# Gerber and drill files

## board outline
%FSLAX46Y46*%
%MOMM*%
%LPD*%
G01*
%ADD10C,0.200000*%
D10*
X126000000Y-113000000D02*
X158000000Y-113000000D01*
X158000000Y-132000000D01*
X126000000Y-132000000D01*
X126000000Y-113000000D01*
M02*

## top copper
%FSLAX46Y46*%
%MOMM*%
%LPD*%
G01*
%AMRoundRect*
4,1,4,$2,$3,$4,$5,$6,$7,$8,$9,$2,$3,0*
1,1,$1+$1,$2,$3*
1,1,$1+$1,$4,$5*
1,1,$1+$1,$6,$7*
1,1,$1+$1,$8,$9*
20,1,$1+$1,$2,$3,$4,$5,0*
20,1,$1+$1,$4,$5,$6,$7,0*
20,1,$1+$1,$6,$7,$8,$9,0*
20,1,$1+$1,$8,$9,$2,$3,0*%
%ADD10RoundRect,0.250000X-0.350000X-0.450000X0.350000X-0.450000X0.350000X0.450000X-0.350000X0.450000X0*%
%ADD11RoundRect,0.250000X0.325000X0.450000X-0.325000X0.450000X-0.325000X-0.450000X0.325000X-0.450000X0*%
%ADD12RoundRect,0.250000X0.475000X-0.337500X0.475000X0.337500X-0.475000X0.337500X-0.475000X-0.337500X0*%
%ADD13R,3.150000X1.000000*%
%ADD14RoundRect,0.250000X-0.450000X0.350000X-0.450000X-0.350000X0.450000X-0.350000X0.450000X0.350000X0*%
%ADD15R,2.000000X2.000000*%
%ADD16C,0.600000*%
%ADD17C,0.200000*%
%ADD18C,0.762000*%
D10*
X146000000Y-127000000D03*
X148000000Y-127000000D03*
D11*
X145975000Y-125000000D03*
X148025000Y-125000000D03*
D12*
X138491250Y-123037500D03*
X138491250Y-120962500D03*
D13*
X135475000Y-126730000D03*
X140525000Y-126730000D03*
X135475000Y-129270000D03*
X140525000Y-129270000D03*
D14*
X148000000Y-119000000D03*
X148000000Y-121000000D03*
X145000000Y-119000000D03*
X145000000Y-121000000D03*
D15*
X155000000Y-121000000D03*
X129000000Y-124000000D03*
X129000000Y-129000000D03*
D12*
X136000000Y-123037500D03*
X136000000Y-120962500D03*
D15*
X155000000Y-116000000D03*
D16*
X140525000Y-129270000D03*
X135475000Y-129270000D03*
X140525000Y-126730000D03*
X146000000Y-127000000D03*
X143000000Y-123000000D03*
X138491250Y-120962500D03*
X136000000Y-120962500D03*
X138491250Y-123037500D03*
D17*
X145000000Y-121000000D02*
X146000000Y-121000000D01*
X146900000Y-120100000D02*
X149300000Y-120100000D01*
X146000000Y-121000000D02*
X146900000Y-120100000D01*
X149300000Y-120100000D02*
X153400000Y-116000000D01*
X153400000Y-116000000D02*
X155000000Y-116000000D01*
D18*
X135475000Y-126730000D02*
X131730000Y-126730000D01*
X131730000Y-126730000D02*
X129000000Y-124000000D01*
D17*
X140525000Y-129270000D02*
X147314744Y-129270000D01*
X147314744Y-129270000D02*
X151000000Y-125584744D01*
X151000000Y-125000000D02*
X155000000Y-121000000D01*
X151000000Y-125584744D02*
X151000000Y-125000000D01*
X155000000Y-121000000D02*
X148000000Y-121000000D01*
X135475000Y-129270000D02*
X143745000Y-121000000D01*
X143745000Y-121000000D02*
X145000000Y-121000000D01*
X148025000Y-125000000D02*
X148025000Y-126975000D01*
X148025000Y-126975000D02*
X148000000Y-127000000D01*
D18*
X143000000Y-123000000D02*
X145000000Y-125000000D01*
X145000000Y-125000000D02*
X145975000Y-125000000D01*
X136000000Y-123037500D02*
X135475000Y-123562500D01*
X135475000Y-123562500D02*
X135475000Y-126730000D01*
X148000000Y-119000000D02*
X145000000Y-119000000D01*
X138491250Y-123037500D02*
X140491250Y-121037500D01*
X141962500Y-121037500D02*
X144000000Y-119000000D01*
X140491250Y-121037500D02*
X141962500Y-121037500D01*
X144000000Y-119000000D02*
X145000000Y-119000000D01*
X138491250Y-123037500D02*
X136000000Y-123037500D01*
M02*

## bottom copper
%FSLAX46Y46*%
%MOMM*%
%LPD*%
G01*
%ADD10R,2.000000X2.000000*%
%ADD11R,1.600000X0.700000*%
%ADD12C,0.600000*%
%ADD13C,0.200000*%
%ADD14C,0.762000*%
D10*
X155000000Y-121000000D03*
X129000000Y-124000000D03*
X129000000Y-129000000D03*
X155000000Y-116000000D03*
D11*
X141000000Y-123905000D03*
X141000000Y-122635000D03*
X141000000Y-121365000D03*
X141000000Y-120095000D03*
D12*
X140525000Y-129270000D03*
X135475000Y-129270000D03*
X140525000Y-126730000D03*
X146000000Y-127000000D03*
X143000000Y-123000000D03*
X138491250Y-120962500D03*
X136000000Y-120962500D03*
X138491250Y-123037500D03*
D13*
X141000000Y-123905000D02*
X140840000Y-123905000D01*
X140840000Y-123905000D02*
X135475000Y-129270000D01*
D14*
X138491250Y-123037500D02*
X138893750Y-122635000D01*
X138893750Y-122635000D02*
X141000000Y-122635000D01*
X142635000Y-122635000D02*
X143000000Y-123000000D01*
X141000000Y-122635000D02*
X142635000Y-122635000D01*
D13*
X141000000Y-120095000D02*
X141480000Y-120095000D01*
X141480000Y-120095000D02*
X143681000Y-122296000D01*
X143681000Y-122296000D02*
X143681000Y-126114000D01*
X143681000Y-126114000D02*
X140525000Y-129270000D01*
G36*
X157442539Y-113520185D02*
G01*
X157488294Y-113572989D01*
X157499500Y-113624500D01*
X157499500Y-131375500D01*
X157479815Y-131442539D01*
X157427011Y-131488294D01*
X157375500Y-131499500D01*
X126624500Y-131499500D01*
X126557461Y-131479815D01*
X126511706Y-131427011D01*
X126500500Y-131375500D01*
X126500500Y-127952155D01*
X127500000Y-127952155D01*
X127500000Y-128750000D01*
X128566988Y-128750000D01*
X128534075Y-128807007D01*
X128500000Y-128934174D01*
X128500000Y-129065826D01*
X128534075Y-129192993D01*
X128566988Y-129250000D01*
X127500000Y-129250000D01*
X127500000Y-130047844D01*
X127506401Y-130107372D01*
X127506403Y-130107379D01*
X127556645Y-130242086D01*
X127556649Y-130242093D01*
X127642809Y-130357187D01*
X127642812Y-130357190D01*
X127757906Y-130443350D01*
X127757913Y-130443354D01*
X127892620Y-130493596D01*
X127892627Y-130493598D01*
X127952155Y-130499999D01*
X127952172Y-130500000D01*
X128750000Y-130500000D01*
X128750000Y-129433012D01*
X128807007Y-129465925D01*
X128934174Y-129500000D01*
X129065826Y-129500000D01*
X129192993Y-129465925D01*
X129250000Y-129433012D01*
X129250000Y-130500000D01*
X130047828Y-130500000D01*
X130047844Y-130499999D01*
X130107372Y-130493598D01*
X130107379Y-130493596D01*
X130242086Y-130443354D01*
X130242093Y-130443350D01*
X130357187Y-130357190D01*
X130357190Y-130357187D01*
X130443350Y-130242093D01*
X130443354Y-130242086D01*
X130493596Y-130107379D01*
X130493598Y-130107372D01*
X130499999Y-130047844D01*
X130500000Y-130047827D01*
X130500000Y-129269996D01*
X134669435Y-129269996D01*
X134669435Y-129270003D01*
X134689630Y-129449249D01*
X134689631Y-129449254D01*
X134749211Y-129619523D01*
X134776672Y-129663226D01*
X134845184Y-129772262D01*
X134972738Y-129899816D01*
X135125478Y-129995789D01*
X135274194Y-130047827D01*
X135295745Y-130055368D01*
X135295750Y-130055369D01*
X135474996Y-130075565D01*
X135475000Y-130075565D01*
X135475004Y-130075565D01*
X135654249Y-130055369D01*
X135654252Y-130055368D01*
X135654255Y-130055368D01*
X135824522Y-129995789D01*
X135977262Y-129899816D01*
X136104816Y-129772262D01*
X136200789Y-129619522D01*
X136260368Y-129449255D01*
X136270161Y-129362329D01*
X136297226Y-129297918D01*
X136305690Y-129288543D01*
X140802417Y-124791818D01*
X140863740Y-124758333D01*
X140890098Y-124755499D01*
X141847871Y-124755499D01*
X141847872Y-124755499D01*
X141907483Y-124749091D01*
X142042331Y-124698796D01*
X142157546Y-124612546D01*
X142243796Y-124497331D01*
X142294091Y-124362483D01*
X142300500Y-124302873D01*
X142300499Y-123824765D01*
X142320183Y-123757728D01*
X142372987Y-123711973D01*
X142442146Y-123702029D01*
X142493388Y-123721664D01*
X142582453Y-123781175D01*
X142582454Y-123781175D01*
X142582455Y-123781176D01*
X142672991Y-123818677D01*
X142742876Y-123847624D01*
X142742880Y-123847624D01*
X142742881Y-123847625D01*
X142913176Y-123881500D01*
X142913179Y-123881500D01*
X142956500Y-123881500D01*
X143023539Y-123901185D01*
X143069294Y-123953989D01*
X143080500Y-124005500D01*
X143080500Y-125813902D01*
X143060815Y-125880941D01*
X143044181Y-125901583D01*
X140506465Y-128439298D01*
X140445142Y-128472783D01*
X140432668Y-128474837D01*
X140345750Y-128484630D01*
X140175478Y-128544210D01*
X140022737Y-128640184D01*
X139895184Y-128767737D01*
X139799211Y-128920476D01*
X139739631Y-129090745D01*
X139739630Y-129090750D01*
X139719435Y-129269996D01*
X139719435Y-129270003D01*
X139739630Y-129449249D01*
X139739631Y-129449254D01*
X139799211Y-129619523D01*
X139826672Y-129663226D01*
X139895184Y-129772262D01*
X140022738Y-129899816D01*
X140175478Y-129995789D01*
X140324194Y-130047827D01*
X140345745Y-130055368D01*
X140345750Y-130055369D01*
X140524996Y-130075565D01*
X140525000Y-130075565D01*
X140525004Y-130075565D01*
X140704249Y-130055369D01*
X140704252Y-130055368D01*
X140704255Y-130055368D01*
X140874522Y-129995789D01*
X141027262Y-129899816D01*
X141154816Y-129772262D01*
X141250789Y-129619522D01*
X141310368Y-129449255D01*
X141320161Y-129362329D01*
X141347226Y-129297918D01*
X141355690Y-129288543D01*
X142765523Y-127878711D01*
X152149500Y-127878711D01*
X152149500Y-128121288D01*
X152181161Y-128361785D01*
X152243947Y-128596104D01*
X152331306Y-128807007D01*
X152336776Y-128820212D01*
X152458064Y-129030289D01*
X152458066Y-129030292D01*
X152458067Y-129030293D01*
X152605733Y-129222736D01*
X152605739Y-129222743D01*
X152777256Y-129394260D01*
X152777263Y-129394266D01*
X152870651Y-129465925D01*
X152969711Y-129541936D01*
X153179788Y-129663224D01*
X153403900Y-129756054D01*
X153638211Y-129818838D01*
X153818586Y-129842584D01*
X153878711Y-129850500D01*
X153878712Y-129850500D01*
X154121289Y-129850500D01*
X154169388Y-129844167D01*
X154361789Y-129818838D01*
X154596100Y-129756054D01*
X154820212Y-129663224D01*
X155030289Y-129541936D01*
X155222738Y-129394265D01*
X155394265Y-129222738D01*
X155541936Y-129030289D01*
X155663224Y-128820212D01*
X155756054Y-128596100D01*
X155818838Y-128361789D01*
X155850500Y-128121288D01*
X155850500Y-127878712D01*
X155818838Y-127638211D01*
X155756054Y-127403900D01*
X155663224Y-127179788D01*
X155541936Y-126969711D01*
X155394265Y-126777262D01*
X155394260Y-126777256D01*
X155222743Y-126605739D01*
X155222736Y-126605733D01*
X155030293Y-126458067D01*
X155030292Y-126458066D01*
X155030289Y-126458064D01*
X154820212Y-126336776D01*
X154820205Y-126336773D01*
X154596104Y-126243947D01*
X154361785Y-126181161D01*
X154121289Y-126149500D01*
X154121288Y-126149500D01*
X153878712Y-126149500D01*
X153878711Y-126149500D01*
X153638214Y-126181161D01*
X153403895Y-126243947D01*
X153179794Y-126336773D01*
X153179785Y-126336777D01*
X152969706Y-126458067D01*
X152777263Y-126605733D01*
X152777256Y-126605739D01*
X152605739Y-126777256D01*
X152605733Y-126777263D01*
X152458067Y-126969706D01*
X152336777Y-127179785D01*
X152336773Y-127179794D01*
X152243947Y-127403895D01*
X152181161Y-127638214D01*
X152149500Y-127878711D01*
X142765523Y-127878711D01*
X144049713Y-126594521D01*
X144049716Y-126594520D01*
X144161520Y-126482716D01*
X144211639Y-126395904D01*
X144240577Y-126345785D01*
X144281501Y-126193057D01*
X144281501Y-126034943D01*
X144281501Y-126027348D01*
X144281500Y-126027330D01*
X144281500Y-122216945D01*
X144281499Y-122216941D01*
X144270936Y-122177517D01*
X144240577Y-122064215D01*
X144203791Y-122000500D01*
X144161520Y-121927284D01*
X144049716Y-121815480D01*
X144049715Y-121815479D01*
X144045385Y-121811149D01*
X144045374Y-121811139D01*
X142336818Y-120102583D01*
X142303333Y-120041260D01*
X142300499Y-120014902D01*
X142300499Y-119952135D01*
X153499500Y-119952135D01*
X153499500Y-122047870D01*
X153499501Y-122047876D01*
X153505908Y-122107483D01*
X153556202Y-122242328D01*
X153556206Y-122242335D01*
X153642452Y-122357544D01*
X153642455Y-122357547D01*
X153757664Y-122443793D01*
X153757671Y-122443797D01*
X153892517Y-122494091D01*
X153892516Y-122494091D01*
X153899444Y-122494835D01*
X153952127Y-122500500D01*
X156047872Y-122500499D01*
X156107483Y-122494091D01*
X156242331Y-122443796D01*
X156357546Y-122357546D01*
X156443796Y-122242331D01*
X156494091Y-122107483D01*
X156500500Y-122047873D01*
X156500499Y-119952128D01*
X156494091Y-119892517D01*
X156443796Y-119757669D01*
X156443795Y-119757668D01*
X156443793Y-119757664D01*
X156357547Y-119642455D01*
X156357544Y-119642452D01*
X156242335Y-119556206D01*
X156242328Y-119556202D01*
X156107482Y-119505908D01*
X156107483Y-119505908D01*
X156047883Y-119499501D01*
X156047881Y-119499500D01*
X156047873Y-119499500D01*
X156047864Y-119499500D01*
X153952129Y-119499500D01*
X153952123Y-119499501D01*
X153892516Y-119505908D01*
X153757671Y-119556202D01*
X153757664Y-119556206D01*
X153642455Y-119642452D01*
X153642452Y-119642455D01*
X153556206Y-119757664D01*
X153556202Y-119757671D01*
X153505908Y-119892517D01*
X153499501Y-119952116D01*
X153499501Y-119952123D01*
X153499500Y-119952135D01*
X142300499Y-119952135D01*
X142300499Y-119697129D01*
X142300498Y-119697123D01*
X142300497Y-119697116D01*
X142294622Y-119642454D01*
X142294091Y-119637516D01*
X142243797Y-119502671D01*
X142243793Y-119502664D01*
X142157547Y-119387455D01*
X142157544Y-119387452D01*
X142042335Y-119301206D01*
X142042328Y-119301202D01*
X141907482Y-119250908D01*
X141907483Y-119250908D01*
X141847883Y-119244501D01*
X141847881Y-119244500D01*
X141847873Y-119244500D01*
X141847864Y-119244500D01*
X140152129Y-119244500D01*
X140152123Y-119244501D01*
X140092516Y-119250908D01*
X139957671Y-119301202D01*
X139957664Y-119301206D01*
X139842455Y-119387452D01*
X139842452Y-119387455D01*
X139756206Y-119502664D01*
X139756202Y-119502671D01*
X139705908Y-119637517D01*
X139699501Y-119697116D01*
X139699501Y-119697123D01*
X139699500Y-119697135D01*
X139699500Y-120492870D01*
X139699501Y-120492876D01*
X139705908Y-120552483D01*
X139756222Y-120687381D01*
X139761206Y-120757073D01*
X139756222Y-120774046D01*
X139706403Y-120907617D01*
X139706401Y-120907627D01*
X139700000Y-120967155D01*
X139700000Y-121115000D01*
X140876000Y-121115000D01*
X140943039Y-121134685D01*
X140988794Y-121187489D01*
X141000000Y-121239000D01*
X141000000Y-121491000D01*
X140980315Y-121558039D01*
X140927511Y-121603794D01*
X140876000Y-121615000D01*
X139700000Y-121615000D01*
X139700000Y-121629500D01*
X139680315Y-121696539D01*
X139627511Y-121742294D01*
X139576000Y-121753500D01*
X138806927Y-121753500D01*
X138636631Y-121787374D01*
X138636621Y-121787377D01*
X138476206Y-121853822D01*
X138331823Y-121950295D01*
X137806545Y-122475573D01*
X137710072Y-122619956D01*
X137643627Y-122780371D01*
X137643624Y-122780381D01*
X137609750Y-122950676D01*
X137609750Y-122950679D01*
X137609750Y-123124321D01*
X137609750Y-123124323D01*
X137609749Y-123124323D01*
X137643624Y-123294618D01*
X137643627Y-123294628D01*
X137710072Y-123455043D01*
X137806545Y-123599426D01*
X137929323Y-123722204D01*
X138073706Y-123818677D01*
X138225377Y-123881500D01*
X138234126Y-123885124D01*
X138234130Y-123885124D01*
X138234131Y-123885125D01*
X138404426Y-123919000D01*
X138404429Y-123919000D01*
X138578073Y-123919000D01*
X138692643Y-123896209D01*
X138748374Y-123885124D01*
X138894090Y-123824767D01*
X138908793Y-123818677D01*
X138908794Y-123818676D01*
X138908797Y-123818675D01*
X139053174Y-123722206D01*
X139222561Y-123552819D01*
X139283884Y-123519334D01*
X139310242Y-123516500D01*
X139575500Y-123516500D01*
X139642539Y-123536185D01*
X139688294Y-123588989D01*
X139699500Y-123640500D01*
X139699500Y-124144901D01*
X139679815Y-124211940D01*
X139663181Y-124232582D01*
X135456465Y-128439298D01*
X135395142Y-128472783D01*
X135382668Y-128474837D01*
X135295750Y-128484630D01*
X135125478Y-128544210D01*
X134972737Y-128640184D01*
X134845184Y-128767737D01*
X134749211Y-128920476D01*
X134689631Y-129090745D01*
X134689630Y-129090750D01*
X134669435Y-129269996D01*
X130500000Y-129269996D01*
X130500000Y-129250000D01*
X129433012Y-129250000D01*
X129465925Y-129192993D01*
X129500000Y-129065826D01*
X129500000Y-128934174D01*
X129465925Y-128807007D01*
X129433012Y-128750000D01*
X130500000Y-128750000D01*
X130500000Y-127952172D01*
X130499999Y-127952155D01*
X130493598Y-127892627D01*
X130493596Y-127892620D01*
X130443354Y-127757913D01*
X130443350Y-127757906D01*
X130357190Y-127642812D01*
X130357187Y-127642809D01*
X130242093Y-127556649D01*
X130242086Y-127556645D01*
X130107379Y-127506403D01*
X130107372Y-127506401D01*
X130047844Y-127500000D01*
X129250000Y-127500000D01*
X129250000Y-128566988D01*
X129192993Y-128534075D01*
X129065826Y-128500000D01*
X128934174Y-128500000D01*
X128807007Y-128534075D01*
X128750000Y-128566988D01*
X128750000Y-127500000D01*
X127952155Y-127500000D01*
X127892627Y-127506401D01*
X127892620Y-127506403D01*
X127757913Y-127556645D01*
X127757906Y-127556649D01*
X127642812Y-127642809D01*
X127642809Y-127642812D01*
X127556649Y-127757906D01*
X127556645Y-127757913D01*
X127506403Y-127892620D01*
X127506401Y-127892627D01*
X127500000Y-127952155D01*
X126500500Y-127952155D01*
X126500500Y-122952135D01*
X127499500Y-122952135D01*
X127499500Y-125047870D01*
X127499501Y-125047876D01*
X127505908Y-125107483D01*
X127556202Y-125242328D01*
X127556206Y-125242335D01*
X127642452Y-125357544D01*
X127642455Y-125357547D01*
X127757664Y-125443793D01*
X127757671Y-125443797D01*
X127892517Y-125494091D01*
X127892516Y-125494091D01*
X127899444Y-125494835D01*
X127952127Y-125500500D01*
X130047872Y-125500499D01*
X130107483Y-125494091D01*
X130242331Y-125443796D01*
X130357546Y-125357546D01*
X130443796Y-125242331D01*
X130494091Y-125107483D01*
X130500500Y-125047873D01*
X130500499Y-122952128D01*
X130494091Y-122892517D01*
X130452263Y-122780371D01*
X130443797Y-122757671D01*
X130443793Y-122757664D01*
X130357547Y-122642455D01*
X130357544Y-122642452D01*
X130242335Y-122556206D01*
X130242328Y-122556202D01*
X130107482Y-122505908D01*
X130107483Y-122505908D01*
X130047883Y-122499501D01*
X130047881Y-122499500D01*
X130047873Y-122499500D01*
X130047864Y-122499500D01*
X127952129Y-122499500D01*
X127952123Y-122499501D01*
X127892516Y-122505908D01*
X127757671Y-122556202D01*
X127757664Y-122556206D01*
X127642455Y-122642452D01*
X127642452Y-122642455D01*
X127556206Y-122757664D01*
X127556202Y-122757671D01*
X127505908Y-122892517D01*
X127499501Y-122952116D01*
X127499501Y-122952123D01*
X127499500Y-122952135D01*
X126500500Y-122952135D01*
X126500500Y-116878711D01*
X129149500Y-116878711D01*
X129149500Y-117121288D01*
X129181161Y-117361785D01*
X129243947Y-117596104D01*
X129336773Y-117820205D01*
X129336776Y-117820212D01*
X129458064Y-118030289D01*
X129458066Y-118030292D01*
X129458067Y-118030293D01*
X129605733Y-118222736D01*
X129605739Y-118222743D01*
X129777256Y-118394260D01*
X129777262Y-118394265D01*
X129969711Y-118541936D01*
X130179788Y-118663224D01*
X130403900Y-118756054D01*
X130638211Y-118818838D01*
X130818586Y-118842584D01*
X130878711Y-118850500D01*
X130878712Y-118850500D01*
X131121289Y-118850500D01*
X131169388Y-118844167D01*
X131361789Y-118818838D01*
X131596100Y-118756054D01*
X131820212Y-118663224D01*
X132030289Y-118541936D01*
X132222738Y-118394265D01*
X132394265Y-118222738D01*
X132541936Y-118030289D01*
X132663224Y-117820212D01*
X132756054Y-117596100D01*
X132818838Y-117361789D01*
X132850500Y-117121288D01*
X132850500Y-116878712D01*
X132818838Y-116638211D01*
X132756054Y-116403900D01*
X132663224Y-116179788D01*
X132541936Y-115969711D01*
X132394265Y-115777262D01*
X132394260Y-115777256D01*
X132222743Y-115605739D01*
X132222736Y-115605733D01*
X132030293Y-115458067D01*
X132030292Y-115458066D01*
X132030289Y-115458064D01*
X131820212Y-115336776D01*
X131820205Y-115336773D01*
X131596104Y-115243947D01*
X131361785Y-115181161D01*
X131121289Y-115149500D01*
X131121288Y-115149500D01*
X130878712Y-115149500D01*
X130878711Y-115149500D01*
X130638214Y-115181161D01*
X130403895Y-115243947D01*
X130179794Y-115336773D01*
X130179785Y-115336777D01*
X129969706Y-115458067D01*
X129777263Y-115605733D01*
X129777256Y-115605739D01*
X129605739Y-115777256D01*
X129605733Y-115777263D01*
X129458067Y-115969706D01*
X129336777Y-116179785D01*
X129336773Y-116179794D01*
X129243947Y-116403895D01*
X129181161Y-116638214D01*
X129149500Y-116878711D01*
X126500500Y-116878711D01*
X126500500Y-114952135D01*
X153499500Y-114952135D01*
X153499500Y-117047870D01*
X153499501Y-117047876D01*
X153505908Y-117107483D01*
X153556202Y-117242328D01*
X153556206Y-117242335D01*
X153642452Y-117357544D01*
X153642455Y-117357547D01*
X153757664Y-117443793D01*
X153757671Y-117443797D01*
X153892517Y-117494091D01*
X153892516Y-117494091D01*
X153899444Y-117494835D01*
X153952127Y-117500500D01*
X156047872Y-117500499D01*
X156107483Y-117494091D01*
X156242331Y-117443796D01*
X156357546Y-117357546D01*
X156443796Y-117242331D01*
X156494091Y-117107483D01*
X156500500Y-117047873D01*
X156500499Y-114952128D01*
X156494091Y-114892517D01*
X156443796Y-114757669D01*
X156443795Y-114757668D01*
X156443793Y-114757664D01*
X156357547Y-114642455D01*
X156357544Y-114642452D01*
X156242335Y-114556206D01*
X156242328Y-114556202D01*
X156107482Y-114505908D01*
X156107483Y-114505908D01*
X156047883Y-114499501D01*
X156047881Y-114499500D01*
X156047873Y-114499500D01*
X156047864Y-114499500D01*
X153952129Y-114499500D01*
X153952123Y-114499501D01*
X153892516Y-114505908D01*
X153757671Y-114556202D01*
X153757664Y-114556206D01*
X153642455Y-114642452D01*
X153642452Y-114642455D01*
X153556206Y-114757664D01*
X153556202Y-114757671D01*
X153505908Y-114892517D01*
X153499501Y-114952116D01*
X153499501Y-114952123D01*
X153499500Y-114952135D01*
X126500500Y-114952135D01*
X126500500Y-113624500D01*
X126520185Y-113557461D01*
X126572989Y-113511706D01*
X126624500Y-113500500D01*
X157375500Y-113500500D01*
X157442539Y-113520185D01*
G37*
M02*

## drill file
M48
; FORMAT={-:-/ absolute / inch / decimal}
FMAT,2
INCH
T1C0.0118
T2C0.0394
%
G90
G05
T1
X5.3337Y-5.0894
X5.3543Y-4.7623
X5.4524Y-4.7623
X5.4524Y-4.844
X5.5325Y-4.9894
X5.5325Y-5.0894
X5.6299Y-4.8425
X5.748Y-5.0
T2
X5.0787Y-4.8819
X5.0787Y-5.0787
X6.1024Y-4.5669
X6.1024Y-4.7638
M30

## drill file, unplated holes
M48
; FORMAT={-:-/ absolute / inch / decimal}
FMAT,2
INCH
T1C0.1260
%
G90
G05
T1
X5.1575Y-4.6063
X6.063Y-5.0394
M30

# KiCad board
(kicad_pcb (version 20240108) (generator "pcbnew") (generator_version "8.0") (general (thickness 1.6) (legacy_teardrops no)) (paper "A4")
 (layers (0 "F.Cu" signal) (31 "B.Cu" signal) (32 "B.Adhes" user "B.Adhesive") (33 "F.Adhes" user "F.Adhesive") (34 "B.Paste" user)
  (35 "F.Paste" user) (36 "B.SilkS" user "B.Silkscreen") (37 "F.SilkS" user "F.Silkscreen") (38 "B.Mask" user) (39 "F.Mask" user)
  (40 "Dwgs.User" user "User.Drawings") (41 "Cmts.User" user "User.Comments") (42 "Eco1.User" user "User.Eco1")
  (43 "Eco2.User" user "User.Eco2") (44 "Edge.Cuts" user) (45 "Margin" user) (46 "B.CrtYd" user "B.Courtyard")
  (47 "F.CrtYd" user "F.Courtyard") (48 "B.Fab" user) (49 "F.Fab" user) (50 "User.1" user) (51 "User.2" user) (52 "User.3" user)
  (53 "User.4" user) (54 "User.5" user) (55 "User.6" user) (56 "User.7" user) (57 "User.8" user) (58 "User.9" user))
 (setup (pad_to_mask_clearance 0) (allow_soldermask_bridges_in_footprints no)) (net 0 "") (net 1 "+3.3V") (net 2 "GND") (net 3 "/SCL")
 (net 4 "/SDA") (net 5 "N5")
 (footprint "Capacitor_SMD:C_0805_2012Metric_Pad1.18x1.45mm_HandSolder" (layer "F.Cu") (at 138.49125 122 90)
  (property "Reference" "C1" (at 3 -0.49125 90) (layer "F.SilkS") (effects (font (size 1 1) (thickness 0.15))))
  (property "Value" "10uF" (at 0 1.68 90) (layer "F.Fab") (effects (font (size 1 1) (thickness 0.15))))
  (pad "1" smd roundrect (at -1.0375 0 90) (size 1.175 1.45) (layers "F.Cu" "F.Paste" "F.Mask") (roundrect_rratio 0.212766) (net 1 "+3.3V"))
  (pad "2" smd roundrect (at 1.0375 0 90) (size 1.175 1.45) (layers "F.Cu" "F.Paste" "F.Mask") (roundrect_rratio 0.212766) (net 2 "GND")))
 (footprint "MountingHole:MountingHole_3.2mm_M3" (layer "F.Cu") (at 131 117)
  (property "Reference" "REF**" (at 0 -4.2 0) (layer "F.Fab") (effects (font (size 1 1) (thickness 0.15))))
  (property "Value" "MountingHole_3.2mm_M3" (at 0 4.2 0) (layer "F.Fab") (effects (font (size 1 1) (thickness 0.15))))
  (pad "" np_thru_hole circle (at 0 0) (size 3.2 3.2) (drill 3.2) (layers "*.Cu" "*.Mask")))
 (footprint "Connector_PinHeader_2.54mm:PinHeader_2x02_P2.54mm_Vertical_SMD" (layer "F.Cu") (at 138 128)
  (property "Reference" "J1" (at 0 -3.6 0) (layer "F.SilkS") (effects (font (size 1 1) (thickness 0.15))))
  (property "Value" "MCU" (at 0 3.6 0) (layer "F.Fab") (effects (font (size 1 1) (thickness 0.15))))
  (pad "1" smd rect (at -2.525 -1.27) (size 3.15 1) (layers "F.Cu" "F.Paste" "F.Mask") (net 1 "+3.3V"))
  (pad "2" smd rect (at 2.525 -1.27) (size 3.15 1) (layers "F.Cu" "F.Paste" "F.Mask") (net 2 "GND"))
  (pad "3" smd rect (at -2.525 1.27) (size 3.15 1) (layers "F.Cu" "F.Paste" "F.Mask") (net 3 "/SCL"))
  (pad "4" smd rect (at 2.525 1.27) (size 3.15 1) (layers "F.Cu" "F.Paste" "F.Mask") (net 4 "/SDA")))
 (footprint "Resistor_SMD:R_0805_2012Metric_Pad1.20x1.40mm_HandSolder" (layer "F.Cu") (at 148 120 -90)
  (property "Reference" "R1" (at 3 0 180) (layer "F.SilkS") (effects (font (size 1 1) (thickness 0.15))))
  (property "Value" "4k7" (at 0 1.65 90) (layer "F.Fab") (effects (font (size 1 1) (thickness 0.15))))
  (pad "1" smd roundrect (at -1 0 270) (size 1.2 1.4) (layers "F.Cu" "F.Paste" "F.Mask") (roundrect_rratio 0.208333) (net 1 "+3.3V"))
  (pad "2" smd roundrect (at 1 0 270) (size 1.2 1.4) (layers "F.Cu" "F.Paste" "F.Mask") (roundrect_rratio 0.208333) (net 4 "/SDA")))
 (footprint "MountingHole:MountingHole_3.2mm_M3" (layer "F.Cu") (at 154 128)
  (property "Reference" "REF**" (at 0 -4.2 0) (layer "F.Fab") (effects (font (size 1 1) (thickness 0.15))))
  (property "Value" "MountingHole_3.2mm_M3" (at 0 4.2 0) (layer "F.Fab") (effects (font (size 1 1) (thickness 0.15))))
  (pad "" np_thru_hole circle (at 0 0) (size 3.2 3.2) (drill 3.2) (layers "*.Cu" "*.Mask")))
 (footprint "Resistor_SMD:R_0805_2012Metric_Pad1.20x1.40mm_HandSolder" (layer "F.Cu") (at 145 120 -90)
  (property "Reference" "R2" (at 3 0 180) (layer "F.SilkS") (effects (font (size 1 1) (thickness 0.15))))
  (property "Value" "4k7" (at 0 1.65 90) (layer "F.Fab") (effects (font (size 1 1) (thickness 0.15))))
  (pad "1" smd roundrect (at -1 0 270) (size 1.2 1.4) (layers "F.Cu" "F.Paste" "F.Mask") (roundrect_rratio 0.208333) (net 1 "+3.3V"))
  (pad "2" smd roundrect (at 1 0 270) (size 1.2 1.4) (layers "F.Cu" "F.Paste" "F.Mask") (roundrect_rratio 0.208333) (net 3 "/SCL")))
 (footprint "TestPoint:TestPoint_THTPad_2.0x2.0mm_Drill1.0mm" (layer "F.Cu") (at 155 121)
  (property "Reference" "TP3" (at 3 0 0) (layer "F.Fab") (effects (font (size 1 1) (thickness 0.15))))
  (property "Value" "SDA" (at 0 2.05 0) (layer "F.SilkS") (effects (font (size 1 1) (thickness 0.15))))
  (pad "1" thru_hole rect (at 0 0) (size 2 2) (drill 1) (layers "*.Cu" "*.Mask") (remove_unused_layers no) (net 4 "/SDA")))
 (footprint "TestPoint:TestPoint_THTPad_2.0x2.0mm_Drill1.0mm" (layer "F.Cu") (at 129 124)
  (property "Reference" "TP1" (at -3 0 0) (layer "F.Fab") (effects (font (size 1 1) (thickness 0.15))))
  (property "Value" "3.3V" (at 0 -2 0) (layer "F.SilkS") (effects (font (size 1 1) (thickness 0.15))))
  (pad "1" thru_hole rect (at 0 0) (size 2 2) (drill 1) (layers "*.Cu" "*.Mask") (remove_unused_layers no) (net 1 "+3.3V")))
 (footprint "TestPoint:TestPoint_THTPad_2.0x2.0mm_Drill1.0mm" (layer "F.Cu") (at 129 129)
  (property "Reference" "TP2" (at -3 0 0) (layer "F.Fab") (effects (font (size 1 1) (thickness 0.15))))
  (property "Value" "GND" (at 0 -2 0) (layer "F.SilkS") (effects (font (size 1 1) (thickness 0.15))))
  (pad "1" thru_hole rect (at 0 0) (size 2 2) (drill 1) (layers "*.Cu" "*.Mask") (remove_unused_layers no) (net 2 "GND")))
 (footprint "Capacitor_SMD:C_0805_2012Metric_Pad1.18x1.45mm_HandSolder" (layer "F.Cu") (at 136 122 90)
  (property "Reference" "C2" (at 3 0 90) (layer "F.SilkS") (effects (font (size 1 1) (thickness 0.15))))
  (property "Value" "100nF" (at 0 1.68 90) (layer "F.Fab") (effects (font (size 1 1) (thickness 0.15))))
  (pad "1" smd roundrect (at -1.0375 0 90) (size 1.175 1.45) (layers "F.Cu" "F.Paste" "F.Mask") (roundrect_rratio 0.212766) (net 1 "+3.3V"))
  (pad "2" smd roundrect (at 1.0375 0 90) (size 1.175 1.45) (layers "F.Cu" "F.Paste" "F.Mask") (roundrect_rratio 0.212766) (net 2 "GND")))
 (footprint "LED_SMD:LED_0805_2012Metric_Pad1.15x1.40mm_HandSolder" (layer "F.Cu") (at 147 125 180)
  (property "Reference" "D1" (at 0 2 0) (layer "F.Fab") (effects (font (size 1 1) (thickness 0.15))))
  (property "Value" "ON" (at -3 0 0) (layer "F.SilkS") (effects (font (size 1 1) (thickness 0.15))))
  (pad "1" smd roundrect (at -1.025 0 180) (size 1.15 1.4) (layers "F.Cu" "F.Paste" "F.Mask") (roundrect_rratio 0.217391) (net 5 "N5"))
  (pad "2" smd roundrect (at 1.025 0 180) (size 1.15 1.4) (layers "F.Cu" "F.Paste" "F.Mask") (roundrect_rratio 0.217391) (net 1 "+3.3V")))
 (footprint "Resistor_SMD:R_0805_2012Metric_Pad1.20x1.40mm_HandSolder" (layer "F.Cu") (at 147 127)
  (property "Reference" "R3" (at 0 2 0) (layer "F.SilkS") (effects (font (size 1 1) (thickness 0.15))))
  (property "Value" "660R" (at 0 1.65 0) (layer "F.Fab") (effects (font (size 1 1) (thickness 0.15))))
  (pad "1" smd roundrect (at -1 0) (size 1.2 1.4) (layers "F.Cu" "F.Paste" "F.Mask") (roundrect_rratio 0.208333) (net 2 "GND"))
  (pad "2" smd roundrect (at 1 0) (size 1.2 1.4) (layers "F.Cu" "F.Paste" "F.Mask") (roundrect_rratio 0.208333) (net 5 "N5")))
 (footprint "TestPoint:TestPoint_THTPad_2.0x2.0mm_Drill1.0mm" (layer "F.Cu") (at 155 116)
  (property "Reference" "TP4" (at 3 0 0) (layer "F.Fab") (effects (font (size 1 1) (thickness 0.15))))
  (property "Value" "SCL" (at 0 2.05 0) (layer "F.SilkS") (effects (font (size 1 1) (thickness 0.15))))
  (pad "1" thru_hole rect (at 0 0) (size 2 2) (drill 1) (layers "*.Cu" "*.Mask") (remove_unused_layers no) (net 3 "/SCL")))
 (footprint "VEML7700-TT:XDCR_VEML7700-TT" (layer "B.Cu") (at 141.9 122)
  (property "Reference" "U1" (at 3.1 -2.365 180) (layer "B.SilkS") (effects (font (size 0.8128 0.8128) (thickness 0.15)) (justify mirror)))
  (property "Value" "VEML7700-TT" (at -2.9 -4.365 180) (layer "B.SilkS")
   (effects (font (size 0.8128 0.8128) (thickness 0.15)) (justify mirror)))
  (pad "1" smd rect (at -0.9 1.905) (size 1.6 0.7) (layers "B.Cu" "B.Paste" "B.Mask") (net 3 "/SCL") (solder_mask_margin 0.102))
  (pad "2" smd rect (at -0.9 0.635) (size 1.6 0.7) (layers "B.Cu" "B.Paste" "B.Mask") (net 1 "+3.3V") (solder_mask_margin 0.102))
  (pad "3" smd rect (at -0.9 -0.635) (size 1.6 0.7) (layers "B.Cu" "B.Paste" "B.Mask") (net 2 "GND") (solder_mask_margin 0.102))
  (pad "4" smd rect (at -0.9 -1.905) (size 1.6 0.7) (layers "B.Cu" "B.Paste" "B.Mask") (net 4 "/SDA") (solder_mask_margin 0.102)))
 (gr_rect (start 126 113) (end 158 132) (stroke (width 0.2) (type default)) (fill none) (layer "Edge.Cuts"))
 (via (at 140.525 126.73) (size 0.6) (drill 0.3) (layers "F.Cu" "B.Cu") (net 2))
 (via (at 138.49125 120.9625) (size 0.6) (drill 0.3) (layers "F.Cu" "B.Cu") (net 2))
 (via (at 146 127) (size 0.6) (drill 0.3) (layers "F.Cu" "B.Cu") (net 2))
 (via (at 136 120.9625) (size 0.6) (drill 0.3) (layers "F.Cu" "B.Cu") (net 2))
 (segment (start 135.475 123.5625) (end 135.475 126.73) (width 0.762) (layer "F.Cu") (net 1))
 (segment (start 136 123.0375) (end 135.475 123.5625) (width 0.762) (layer "F.Cu") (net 1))
 (segment (start 135.475 126.73) (end 131.73 126.73) (width 0.762) (layer "F.Cu") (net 1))
 (segment (start 144 119) (end 145 119) (width 0.762) (layer "F.Cu") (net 1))
 (segment (start 138.49125 123.0375) (end 140.49125 121.0375) (width 0.762) (layer "F.Cu") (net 1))
 (segment (start 148 119) (end 145 119) (width 0.762) (layer "F.Cu") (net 1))
 (segment (start 143 123) (end 145 125) (width 0.762) (layer "F.Cu") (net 1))
 (segment (start 141.9625 121.0375) (end 144 119) (width 0.762) (layer "F.Cu") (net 1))
 (segment (start 138.49125 123.0375) (end 136 123.0375) (width 0.762) (layer "F.Cu") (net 1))
 (segment (start 140.49125 121.0375) (end 141.9625 121.0375) (width 0.762) (layer "F.Cu") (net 1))
 (segment (start 145 125) (end 145.975 125) (width 0.762) (layer "F.Cu") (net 1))
 (segment (start 131.73 126.73) (end 129 124) (width 0.762) (layer "F.Cu") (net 1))
 (via (at 138.49125 123.0375) (size 0.6) (drill 0.3) (layers "F.Cu" "B.Cu") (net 1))
 (via (at 143 123) (size 0.6) (drill 0.3) (layers "F.Cu" "B.Cu") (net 1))
 (segment (start 138.49125 123.0375) (end 138.89375 122.635) (width 0.762) (layer "B.Cu") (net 1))
 (segment (start 142.635 122.635) (end 143 123) (width 0.762) (layer "B.Cu") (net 1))
 (segment (start 141 122.635) (end 142.635 122.635) (width 0.762) (layer "B.Cu") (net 1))
 (segment (start 138.89375 122.635) (end 141 122.635) (width 0.762) (layer "B.Cu") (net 1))
 (segment (start 148.025 126.975) (end 148 127) (width 0.2) (layer "F.Cu") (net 5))
 (segment (start 148.025 125) (end 148.025 126.975) (width 0.2) (layer "F.Cu") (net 5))
 (segment (start 140.525 129.27) (end 147.314744 129.27) (width 0.2) (layer "F.Cu") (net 4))
 (segment (start 155 121) (end 148 121) (width 0.2) (layer "F.Cu") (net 4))
 (segment (start 147.314744 129.27) (end 151 125.584744) (width 0.2) (layer "F.Cu") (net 4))
 (segment (start 151 125) (end 155 121) (width 0.2) (layer "F.Cu") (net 4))
 (segment (start 151 125.584744) (end 151 125) (width 0.2) (layer "F.Cu") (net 4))
 (via (at 140.525 129.27) (size 0.6) (drill 0.3) (layers "F.Cu" "B.Cu") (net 4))
 (segment (start 143.681 126.114) (end 140.525 129.27) (width 0.2) (layer "B.Cu") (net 4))
 (segment (start 141 120.095) (end 141.48 120.095) (width 0.2) (layer "B.Cu") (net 4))
 (segment (start 143.681 122.296) (end 143.681 126.114) (width 0.2) (layer "B.Cu") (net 4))
 (segment (start 141.48 120.095) (end 143.681 122.296) (width 0.2) (layer "B.Cu") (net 4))
 (segment (start 146.9 120.1) (end 149.3 120.1) (width 0.2) (layer "F.Cu") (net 3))
 (segment (start 143.745 121) (end 145 121) (width 0.2) (layer "F.Cu") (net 3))
 (segment (start 153.4 116) (end 155 116) (width 0.2) (layer "F.Cu") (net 3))
 (segment (start 146 121) (end 146.9 120.1) (width 0.2) (layer "F.Cu") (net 3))
 (segment (start 145 121) (end 146 121) (width 0.2) (layer "F.Cu") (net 3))
 (segment (start 135.475 129.27) (end 143.745 121) (width 0.2) (layer "F.Cu") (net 3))
 (segment (start 149.3 120.1) (end 153.4 116) (width 0.2) (layer "F.Cu") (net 3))
 (via (at 135.475 129.27) (size 0.6) (drill 0.3) (layers "F.Cu" "B.Cu") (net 3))
 (segment (start 140.84 123.905) (end 135.475 129.27) (width 0.2) (layer "B.Cu") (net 3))
 (segment (start 141 123.905) (end 140.84 123.905) (width 0.2) (layer "B.Cu") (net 3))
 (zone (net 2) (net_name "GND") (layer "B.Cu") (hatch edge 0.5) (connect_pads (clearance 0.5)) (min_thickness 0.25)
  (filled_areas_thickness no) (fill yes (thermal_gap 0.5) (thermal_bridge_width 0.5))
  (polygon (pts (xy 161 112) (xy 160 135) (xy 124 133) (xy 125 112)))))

